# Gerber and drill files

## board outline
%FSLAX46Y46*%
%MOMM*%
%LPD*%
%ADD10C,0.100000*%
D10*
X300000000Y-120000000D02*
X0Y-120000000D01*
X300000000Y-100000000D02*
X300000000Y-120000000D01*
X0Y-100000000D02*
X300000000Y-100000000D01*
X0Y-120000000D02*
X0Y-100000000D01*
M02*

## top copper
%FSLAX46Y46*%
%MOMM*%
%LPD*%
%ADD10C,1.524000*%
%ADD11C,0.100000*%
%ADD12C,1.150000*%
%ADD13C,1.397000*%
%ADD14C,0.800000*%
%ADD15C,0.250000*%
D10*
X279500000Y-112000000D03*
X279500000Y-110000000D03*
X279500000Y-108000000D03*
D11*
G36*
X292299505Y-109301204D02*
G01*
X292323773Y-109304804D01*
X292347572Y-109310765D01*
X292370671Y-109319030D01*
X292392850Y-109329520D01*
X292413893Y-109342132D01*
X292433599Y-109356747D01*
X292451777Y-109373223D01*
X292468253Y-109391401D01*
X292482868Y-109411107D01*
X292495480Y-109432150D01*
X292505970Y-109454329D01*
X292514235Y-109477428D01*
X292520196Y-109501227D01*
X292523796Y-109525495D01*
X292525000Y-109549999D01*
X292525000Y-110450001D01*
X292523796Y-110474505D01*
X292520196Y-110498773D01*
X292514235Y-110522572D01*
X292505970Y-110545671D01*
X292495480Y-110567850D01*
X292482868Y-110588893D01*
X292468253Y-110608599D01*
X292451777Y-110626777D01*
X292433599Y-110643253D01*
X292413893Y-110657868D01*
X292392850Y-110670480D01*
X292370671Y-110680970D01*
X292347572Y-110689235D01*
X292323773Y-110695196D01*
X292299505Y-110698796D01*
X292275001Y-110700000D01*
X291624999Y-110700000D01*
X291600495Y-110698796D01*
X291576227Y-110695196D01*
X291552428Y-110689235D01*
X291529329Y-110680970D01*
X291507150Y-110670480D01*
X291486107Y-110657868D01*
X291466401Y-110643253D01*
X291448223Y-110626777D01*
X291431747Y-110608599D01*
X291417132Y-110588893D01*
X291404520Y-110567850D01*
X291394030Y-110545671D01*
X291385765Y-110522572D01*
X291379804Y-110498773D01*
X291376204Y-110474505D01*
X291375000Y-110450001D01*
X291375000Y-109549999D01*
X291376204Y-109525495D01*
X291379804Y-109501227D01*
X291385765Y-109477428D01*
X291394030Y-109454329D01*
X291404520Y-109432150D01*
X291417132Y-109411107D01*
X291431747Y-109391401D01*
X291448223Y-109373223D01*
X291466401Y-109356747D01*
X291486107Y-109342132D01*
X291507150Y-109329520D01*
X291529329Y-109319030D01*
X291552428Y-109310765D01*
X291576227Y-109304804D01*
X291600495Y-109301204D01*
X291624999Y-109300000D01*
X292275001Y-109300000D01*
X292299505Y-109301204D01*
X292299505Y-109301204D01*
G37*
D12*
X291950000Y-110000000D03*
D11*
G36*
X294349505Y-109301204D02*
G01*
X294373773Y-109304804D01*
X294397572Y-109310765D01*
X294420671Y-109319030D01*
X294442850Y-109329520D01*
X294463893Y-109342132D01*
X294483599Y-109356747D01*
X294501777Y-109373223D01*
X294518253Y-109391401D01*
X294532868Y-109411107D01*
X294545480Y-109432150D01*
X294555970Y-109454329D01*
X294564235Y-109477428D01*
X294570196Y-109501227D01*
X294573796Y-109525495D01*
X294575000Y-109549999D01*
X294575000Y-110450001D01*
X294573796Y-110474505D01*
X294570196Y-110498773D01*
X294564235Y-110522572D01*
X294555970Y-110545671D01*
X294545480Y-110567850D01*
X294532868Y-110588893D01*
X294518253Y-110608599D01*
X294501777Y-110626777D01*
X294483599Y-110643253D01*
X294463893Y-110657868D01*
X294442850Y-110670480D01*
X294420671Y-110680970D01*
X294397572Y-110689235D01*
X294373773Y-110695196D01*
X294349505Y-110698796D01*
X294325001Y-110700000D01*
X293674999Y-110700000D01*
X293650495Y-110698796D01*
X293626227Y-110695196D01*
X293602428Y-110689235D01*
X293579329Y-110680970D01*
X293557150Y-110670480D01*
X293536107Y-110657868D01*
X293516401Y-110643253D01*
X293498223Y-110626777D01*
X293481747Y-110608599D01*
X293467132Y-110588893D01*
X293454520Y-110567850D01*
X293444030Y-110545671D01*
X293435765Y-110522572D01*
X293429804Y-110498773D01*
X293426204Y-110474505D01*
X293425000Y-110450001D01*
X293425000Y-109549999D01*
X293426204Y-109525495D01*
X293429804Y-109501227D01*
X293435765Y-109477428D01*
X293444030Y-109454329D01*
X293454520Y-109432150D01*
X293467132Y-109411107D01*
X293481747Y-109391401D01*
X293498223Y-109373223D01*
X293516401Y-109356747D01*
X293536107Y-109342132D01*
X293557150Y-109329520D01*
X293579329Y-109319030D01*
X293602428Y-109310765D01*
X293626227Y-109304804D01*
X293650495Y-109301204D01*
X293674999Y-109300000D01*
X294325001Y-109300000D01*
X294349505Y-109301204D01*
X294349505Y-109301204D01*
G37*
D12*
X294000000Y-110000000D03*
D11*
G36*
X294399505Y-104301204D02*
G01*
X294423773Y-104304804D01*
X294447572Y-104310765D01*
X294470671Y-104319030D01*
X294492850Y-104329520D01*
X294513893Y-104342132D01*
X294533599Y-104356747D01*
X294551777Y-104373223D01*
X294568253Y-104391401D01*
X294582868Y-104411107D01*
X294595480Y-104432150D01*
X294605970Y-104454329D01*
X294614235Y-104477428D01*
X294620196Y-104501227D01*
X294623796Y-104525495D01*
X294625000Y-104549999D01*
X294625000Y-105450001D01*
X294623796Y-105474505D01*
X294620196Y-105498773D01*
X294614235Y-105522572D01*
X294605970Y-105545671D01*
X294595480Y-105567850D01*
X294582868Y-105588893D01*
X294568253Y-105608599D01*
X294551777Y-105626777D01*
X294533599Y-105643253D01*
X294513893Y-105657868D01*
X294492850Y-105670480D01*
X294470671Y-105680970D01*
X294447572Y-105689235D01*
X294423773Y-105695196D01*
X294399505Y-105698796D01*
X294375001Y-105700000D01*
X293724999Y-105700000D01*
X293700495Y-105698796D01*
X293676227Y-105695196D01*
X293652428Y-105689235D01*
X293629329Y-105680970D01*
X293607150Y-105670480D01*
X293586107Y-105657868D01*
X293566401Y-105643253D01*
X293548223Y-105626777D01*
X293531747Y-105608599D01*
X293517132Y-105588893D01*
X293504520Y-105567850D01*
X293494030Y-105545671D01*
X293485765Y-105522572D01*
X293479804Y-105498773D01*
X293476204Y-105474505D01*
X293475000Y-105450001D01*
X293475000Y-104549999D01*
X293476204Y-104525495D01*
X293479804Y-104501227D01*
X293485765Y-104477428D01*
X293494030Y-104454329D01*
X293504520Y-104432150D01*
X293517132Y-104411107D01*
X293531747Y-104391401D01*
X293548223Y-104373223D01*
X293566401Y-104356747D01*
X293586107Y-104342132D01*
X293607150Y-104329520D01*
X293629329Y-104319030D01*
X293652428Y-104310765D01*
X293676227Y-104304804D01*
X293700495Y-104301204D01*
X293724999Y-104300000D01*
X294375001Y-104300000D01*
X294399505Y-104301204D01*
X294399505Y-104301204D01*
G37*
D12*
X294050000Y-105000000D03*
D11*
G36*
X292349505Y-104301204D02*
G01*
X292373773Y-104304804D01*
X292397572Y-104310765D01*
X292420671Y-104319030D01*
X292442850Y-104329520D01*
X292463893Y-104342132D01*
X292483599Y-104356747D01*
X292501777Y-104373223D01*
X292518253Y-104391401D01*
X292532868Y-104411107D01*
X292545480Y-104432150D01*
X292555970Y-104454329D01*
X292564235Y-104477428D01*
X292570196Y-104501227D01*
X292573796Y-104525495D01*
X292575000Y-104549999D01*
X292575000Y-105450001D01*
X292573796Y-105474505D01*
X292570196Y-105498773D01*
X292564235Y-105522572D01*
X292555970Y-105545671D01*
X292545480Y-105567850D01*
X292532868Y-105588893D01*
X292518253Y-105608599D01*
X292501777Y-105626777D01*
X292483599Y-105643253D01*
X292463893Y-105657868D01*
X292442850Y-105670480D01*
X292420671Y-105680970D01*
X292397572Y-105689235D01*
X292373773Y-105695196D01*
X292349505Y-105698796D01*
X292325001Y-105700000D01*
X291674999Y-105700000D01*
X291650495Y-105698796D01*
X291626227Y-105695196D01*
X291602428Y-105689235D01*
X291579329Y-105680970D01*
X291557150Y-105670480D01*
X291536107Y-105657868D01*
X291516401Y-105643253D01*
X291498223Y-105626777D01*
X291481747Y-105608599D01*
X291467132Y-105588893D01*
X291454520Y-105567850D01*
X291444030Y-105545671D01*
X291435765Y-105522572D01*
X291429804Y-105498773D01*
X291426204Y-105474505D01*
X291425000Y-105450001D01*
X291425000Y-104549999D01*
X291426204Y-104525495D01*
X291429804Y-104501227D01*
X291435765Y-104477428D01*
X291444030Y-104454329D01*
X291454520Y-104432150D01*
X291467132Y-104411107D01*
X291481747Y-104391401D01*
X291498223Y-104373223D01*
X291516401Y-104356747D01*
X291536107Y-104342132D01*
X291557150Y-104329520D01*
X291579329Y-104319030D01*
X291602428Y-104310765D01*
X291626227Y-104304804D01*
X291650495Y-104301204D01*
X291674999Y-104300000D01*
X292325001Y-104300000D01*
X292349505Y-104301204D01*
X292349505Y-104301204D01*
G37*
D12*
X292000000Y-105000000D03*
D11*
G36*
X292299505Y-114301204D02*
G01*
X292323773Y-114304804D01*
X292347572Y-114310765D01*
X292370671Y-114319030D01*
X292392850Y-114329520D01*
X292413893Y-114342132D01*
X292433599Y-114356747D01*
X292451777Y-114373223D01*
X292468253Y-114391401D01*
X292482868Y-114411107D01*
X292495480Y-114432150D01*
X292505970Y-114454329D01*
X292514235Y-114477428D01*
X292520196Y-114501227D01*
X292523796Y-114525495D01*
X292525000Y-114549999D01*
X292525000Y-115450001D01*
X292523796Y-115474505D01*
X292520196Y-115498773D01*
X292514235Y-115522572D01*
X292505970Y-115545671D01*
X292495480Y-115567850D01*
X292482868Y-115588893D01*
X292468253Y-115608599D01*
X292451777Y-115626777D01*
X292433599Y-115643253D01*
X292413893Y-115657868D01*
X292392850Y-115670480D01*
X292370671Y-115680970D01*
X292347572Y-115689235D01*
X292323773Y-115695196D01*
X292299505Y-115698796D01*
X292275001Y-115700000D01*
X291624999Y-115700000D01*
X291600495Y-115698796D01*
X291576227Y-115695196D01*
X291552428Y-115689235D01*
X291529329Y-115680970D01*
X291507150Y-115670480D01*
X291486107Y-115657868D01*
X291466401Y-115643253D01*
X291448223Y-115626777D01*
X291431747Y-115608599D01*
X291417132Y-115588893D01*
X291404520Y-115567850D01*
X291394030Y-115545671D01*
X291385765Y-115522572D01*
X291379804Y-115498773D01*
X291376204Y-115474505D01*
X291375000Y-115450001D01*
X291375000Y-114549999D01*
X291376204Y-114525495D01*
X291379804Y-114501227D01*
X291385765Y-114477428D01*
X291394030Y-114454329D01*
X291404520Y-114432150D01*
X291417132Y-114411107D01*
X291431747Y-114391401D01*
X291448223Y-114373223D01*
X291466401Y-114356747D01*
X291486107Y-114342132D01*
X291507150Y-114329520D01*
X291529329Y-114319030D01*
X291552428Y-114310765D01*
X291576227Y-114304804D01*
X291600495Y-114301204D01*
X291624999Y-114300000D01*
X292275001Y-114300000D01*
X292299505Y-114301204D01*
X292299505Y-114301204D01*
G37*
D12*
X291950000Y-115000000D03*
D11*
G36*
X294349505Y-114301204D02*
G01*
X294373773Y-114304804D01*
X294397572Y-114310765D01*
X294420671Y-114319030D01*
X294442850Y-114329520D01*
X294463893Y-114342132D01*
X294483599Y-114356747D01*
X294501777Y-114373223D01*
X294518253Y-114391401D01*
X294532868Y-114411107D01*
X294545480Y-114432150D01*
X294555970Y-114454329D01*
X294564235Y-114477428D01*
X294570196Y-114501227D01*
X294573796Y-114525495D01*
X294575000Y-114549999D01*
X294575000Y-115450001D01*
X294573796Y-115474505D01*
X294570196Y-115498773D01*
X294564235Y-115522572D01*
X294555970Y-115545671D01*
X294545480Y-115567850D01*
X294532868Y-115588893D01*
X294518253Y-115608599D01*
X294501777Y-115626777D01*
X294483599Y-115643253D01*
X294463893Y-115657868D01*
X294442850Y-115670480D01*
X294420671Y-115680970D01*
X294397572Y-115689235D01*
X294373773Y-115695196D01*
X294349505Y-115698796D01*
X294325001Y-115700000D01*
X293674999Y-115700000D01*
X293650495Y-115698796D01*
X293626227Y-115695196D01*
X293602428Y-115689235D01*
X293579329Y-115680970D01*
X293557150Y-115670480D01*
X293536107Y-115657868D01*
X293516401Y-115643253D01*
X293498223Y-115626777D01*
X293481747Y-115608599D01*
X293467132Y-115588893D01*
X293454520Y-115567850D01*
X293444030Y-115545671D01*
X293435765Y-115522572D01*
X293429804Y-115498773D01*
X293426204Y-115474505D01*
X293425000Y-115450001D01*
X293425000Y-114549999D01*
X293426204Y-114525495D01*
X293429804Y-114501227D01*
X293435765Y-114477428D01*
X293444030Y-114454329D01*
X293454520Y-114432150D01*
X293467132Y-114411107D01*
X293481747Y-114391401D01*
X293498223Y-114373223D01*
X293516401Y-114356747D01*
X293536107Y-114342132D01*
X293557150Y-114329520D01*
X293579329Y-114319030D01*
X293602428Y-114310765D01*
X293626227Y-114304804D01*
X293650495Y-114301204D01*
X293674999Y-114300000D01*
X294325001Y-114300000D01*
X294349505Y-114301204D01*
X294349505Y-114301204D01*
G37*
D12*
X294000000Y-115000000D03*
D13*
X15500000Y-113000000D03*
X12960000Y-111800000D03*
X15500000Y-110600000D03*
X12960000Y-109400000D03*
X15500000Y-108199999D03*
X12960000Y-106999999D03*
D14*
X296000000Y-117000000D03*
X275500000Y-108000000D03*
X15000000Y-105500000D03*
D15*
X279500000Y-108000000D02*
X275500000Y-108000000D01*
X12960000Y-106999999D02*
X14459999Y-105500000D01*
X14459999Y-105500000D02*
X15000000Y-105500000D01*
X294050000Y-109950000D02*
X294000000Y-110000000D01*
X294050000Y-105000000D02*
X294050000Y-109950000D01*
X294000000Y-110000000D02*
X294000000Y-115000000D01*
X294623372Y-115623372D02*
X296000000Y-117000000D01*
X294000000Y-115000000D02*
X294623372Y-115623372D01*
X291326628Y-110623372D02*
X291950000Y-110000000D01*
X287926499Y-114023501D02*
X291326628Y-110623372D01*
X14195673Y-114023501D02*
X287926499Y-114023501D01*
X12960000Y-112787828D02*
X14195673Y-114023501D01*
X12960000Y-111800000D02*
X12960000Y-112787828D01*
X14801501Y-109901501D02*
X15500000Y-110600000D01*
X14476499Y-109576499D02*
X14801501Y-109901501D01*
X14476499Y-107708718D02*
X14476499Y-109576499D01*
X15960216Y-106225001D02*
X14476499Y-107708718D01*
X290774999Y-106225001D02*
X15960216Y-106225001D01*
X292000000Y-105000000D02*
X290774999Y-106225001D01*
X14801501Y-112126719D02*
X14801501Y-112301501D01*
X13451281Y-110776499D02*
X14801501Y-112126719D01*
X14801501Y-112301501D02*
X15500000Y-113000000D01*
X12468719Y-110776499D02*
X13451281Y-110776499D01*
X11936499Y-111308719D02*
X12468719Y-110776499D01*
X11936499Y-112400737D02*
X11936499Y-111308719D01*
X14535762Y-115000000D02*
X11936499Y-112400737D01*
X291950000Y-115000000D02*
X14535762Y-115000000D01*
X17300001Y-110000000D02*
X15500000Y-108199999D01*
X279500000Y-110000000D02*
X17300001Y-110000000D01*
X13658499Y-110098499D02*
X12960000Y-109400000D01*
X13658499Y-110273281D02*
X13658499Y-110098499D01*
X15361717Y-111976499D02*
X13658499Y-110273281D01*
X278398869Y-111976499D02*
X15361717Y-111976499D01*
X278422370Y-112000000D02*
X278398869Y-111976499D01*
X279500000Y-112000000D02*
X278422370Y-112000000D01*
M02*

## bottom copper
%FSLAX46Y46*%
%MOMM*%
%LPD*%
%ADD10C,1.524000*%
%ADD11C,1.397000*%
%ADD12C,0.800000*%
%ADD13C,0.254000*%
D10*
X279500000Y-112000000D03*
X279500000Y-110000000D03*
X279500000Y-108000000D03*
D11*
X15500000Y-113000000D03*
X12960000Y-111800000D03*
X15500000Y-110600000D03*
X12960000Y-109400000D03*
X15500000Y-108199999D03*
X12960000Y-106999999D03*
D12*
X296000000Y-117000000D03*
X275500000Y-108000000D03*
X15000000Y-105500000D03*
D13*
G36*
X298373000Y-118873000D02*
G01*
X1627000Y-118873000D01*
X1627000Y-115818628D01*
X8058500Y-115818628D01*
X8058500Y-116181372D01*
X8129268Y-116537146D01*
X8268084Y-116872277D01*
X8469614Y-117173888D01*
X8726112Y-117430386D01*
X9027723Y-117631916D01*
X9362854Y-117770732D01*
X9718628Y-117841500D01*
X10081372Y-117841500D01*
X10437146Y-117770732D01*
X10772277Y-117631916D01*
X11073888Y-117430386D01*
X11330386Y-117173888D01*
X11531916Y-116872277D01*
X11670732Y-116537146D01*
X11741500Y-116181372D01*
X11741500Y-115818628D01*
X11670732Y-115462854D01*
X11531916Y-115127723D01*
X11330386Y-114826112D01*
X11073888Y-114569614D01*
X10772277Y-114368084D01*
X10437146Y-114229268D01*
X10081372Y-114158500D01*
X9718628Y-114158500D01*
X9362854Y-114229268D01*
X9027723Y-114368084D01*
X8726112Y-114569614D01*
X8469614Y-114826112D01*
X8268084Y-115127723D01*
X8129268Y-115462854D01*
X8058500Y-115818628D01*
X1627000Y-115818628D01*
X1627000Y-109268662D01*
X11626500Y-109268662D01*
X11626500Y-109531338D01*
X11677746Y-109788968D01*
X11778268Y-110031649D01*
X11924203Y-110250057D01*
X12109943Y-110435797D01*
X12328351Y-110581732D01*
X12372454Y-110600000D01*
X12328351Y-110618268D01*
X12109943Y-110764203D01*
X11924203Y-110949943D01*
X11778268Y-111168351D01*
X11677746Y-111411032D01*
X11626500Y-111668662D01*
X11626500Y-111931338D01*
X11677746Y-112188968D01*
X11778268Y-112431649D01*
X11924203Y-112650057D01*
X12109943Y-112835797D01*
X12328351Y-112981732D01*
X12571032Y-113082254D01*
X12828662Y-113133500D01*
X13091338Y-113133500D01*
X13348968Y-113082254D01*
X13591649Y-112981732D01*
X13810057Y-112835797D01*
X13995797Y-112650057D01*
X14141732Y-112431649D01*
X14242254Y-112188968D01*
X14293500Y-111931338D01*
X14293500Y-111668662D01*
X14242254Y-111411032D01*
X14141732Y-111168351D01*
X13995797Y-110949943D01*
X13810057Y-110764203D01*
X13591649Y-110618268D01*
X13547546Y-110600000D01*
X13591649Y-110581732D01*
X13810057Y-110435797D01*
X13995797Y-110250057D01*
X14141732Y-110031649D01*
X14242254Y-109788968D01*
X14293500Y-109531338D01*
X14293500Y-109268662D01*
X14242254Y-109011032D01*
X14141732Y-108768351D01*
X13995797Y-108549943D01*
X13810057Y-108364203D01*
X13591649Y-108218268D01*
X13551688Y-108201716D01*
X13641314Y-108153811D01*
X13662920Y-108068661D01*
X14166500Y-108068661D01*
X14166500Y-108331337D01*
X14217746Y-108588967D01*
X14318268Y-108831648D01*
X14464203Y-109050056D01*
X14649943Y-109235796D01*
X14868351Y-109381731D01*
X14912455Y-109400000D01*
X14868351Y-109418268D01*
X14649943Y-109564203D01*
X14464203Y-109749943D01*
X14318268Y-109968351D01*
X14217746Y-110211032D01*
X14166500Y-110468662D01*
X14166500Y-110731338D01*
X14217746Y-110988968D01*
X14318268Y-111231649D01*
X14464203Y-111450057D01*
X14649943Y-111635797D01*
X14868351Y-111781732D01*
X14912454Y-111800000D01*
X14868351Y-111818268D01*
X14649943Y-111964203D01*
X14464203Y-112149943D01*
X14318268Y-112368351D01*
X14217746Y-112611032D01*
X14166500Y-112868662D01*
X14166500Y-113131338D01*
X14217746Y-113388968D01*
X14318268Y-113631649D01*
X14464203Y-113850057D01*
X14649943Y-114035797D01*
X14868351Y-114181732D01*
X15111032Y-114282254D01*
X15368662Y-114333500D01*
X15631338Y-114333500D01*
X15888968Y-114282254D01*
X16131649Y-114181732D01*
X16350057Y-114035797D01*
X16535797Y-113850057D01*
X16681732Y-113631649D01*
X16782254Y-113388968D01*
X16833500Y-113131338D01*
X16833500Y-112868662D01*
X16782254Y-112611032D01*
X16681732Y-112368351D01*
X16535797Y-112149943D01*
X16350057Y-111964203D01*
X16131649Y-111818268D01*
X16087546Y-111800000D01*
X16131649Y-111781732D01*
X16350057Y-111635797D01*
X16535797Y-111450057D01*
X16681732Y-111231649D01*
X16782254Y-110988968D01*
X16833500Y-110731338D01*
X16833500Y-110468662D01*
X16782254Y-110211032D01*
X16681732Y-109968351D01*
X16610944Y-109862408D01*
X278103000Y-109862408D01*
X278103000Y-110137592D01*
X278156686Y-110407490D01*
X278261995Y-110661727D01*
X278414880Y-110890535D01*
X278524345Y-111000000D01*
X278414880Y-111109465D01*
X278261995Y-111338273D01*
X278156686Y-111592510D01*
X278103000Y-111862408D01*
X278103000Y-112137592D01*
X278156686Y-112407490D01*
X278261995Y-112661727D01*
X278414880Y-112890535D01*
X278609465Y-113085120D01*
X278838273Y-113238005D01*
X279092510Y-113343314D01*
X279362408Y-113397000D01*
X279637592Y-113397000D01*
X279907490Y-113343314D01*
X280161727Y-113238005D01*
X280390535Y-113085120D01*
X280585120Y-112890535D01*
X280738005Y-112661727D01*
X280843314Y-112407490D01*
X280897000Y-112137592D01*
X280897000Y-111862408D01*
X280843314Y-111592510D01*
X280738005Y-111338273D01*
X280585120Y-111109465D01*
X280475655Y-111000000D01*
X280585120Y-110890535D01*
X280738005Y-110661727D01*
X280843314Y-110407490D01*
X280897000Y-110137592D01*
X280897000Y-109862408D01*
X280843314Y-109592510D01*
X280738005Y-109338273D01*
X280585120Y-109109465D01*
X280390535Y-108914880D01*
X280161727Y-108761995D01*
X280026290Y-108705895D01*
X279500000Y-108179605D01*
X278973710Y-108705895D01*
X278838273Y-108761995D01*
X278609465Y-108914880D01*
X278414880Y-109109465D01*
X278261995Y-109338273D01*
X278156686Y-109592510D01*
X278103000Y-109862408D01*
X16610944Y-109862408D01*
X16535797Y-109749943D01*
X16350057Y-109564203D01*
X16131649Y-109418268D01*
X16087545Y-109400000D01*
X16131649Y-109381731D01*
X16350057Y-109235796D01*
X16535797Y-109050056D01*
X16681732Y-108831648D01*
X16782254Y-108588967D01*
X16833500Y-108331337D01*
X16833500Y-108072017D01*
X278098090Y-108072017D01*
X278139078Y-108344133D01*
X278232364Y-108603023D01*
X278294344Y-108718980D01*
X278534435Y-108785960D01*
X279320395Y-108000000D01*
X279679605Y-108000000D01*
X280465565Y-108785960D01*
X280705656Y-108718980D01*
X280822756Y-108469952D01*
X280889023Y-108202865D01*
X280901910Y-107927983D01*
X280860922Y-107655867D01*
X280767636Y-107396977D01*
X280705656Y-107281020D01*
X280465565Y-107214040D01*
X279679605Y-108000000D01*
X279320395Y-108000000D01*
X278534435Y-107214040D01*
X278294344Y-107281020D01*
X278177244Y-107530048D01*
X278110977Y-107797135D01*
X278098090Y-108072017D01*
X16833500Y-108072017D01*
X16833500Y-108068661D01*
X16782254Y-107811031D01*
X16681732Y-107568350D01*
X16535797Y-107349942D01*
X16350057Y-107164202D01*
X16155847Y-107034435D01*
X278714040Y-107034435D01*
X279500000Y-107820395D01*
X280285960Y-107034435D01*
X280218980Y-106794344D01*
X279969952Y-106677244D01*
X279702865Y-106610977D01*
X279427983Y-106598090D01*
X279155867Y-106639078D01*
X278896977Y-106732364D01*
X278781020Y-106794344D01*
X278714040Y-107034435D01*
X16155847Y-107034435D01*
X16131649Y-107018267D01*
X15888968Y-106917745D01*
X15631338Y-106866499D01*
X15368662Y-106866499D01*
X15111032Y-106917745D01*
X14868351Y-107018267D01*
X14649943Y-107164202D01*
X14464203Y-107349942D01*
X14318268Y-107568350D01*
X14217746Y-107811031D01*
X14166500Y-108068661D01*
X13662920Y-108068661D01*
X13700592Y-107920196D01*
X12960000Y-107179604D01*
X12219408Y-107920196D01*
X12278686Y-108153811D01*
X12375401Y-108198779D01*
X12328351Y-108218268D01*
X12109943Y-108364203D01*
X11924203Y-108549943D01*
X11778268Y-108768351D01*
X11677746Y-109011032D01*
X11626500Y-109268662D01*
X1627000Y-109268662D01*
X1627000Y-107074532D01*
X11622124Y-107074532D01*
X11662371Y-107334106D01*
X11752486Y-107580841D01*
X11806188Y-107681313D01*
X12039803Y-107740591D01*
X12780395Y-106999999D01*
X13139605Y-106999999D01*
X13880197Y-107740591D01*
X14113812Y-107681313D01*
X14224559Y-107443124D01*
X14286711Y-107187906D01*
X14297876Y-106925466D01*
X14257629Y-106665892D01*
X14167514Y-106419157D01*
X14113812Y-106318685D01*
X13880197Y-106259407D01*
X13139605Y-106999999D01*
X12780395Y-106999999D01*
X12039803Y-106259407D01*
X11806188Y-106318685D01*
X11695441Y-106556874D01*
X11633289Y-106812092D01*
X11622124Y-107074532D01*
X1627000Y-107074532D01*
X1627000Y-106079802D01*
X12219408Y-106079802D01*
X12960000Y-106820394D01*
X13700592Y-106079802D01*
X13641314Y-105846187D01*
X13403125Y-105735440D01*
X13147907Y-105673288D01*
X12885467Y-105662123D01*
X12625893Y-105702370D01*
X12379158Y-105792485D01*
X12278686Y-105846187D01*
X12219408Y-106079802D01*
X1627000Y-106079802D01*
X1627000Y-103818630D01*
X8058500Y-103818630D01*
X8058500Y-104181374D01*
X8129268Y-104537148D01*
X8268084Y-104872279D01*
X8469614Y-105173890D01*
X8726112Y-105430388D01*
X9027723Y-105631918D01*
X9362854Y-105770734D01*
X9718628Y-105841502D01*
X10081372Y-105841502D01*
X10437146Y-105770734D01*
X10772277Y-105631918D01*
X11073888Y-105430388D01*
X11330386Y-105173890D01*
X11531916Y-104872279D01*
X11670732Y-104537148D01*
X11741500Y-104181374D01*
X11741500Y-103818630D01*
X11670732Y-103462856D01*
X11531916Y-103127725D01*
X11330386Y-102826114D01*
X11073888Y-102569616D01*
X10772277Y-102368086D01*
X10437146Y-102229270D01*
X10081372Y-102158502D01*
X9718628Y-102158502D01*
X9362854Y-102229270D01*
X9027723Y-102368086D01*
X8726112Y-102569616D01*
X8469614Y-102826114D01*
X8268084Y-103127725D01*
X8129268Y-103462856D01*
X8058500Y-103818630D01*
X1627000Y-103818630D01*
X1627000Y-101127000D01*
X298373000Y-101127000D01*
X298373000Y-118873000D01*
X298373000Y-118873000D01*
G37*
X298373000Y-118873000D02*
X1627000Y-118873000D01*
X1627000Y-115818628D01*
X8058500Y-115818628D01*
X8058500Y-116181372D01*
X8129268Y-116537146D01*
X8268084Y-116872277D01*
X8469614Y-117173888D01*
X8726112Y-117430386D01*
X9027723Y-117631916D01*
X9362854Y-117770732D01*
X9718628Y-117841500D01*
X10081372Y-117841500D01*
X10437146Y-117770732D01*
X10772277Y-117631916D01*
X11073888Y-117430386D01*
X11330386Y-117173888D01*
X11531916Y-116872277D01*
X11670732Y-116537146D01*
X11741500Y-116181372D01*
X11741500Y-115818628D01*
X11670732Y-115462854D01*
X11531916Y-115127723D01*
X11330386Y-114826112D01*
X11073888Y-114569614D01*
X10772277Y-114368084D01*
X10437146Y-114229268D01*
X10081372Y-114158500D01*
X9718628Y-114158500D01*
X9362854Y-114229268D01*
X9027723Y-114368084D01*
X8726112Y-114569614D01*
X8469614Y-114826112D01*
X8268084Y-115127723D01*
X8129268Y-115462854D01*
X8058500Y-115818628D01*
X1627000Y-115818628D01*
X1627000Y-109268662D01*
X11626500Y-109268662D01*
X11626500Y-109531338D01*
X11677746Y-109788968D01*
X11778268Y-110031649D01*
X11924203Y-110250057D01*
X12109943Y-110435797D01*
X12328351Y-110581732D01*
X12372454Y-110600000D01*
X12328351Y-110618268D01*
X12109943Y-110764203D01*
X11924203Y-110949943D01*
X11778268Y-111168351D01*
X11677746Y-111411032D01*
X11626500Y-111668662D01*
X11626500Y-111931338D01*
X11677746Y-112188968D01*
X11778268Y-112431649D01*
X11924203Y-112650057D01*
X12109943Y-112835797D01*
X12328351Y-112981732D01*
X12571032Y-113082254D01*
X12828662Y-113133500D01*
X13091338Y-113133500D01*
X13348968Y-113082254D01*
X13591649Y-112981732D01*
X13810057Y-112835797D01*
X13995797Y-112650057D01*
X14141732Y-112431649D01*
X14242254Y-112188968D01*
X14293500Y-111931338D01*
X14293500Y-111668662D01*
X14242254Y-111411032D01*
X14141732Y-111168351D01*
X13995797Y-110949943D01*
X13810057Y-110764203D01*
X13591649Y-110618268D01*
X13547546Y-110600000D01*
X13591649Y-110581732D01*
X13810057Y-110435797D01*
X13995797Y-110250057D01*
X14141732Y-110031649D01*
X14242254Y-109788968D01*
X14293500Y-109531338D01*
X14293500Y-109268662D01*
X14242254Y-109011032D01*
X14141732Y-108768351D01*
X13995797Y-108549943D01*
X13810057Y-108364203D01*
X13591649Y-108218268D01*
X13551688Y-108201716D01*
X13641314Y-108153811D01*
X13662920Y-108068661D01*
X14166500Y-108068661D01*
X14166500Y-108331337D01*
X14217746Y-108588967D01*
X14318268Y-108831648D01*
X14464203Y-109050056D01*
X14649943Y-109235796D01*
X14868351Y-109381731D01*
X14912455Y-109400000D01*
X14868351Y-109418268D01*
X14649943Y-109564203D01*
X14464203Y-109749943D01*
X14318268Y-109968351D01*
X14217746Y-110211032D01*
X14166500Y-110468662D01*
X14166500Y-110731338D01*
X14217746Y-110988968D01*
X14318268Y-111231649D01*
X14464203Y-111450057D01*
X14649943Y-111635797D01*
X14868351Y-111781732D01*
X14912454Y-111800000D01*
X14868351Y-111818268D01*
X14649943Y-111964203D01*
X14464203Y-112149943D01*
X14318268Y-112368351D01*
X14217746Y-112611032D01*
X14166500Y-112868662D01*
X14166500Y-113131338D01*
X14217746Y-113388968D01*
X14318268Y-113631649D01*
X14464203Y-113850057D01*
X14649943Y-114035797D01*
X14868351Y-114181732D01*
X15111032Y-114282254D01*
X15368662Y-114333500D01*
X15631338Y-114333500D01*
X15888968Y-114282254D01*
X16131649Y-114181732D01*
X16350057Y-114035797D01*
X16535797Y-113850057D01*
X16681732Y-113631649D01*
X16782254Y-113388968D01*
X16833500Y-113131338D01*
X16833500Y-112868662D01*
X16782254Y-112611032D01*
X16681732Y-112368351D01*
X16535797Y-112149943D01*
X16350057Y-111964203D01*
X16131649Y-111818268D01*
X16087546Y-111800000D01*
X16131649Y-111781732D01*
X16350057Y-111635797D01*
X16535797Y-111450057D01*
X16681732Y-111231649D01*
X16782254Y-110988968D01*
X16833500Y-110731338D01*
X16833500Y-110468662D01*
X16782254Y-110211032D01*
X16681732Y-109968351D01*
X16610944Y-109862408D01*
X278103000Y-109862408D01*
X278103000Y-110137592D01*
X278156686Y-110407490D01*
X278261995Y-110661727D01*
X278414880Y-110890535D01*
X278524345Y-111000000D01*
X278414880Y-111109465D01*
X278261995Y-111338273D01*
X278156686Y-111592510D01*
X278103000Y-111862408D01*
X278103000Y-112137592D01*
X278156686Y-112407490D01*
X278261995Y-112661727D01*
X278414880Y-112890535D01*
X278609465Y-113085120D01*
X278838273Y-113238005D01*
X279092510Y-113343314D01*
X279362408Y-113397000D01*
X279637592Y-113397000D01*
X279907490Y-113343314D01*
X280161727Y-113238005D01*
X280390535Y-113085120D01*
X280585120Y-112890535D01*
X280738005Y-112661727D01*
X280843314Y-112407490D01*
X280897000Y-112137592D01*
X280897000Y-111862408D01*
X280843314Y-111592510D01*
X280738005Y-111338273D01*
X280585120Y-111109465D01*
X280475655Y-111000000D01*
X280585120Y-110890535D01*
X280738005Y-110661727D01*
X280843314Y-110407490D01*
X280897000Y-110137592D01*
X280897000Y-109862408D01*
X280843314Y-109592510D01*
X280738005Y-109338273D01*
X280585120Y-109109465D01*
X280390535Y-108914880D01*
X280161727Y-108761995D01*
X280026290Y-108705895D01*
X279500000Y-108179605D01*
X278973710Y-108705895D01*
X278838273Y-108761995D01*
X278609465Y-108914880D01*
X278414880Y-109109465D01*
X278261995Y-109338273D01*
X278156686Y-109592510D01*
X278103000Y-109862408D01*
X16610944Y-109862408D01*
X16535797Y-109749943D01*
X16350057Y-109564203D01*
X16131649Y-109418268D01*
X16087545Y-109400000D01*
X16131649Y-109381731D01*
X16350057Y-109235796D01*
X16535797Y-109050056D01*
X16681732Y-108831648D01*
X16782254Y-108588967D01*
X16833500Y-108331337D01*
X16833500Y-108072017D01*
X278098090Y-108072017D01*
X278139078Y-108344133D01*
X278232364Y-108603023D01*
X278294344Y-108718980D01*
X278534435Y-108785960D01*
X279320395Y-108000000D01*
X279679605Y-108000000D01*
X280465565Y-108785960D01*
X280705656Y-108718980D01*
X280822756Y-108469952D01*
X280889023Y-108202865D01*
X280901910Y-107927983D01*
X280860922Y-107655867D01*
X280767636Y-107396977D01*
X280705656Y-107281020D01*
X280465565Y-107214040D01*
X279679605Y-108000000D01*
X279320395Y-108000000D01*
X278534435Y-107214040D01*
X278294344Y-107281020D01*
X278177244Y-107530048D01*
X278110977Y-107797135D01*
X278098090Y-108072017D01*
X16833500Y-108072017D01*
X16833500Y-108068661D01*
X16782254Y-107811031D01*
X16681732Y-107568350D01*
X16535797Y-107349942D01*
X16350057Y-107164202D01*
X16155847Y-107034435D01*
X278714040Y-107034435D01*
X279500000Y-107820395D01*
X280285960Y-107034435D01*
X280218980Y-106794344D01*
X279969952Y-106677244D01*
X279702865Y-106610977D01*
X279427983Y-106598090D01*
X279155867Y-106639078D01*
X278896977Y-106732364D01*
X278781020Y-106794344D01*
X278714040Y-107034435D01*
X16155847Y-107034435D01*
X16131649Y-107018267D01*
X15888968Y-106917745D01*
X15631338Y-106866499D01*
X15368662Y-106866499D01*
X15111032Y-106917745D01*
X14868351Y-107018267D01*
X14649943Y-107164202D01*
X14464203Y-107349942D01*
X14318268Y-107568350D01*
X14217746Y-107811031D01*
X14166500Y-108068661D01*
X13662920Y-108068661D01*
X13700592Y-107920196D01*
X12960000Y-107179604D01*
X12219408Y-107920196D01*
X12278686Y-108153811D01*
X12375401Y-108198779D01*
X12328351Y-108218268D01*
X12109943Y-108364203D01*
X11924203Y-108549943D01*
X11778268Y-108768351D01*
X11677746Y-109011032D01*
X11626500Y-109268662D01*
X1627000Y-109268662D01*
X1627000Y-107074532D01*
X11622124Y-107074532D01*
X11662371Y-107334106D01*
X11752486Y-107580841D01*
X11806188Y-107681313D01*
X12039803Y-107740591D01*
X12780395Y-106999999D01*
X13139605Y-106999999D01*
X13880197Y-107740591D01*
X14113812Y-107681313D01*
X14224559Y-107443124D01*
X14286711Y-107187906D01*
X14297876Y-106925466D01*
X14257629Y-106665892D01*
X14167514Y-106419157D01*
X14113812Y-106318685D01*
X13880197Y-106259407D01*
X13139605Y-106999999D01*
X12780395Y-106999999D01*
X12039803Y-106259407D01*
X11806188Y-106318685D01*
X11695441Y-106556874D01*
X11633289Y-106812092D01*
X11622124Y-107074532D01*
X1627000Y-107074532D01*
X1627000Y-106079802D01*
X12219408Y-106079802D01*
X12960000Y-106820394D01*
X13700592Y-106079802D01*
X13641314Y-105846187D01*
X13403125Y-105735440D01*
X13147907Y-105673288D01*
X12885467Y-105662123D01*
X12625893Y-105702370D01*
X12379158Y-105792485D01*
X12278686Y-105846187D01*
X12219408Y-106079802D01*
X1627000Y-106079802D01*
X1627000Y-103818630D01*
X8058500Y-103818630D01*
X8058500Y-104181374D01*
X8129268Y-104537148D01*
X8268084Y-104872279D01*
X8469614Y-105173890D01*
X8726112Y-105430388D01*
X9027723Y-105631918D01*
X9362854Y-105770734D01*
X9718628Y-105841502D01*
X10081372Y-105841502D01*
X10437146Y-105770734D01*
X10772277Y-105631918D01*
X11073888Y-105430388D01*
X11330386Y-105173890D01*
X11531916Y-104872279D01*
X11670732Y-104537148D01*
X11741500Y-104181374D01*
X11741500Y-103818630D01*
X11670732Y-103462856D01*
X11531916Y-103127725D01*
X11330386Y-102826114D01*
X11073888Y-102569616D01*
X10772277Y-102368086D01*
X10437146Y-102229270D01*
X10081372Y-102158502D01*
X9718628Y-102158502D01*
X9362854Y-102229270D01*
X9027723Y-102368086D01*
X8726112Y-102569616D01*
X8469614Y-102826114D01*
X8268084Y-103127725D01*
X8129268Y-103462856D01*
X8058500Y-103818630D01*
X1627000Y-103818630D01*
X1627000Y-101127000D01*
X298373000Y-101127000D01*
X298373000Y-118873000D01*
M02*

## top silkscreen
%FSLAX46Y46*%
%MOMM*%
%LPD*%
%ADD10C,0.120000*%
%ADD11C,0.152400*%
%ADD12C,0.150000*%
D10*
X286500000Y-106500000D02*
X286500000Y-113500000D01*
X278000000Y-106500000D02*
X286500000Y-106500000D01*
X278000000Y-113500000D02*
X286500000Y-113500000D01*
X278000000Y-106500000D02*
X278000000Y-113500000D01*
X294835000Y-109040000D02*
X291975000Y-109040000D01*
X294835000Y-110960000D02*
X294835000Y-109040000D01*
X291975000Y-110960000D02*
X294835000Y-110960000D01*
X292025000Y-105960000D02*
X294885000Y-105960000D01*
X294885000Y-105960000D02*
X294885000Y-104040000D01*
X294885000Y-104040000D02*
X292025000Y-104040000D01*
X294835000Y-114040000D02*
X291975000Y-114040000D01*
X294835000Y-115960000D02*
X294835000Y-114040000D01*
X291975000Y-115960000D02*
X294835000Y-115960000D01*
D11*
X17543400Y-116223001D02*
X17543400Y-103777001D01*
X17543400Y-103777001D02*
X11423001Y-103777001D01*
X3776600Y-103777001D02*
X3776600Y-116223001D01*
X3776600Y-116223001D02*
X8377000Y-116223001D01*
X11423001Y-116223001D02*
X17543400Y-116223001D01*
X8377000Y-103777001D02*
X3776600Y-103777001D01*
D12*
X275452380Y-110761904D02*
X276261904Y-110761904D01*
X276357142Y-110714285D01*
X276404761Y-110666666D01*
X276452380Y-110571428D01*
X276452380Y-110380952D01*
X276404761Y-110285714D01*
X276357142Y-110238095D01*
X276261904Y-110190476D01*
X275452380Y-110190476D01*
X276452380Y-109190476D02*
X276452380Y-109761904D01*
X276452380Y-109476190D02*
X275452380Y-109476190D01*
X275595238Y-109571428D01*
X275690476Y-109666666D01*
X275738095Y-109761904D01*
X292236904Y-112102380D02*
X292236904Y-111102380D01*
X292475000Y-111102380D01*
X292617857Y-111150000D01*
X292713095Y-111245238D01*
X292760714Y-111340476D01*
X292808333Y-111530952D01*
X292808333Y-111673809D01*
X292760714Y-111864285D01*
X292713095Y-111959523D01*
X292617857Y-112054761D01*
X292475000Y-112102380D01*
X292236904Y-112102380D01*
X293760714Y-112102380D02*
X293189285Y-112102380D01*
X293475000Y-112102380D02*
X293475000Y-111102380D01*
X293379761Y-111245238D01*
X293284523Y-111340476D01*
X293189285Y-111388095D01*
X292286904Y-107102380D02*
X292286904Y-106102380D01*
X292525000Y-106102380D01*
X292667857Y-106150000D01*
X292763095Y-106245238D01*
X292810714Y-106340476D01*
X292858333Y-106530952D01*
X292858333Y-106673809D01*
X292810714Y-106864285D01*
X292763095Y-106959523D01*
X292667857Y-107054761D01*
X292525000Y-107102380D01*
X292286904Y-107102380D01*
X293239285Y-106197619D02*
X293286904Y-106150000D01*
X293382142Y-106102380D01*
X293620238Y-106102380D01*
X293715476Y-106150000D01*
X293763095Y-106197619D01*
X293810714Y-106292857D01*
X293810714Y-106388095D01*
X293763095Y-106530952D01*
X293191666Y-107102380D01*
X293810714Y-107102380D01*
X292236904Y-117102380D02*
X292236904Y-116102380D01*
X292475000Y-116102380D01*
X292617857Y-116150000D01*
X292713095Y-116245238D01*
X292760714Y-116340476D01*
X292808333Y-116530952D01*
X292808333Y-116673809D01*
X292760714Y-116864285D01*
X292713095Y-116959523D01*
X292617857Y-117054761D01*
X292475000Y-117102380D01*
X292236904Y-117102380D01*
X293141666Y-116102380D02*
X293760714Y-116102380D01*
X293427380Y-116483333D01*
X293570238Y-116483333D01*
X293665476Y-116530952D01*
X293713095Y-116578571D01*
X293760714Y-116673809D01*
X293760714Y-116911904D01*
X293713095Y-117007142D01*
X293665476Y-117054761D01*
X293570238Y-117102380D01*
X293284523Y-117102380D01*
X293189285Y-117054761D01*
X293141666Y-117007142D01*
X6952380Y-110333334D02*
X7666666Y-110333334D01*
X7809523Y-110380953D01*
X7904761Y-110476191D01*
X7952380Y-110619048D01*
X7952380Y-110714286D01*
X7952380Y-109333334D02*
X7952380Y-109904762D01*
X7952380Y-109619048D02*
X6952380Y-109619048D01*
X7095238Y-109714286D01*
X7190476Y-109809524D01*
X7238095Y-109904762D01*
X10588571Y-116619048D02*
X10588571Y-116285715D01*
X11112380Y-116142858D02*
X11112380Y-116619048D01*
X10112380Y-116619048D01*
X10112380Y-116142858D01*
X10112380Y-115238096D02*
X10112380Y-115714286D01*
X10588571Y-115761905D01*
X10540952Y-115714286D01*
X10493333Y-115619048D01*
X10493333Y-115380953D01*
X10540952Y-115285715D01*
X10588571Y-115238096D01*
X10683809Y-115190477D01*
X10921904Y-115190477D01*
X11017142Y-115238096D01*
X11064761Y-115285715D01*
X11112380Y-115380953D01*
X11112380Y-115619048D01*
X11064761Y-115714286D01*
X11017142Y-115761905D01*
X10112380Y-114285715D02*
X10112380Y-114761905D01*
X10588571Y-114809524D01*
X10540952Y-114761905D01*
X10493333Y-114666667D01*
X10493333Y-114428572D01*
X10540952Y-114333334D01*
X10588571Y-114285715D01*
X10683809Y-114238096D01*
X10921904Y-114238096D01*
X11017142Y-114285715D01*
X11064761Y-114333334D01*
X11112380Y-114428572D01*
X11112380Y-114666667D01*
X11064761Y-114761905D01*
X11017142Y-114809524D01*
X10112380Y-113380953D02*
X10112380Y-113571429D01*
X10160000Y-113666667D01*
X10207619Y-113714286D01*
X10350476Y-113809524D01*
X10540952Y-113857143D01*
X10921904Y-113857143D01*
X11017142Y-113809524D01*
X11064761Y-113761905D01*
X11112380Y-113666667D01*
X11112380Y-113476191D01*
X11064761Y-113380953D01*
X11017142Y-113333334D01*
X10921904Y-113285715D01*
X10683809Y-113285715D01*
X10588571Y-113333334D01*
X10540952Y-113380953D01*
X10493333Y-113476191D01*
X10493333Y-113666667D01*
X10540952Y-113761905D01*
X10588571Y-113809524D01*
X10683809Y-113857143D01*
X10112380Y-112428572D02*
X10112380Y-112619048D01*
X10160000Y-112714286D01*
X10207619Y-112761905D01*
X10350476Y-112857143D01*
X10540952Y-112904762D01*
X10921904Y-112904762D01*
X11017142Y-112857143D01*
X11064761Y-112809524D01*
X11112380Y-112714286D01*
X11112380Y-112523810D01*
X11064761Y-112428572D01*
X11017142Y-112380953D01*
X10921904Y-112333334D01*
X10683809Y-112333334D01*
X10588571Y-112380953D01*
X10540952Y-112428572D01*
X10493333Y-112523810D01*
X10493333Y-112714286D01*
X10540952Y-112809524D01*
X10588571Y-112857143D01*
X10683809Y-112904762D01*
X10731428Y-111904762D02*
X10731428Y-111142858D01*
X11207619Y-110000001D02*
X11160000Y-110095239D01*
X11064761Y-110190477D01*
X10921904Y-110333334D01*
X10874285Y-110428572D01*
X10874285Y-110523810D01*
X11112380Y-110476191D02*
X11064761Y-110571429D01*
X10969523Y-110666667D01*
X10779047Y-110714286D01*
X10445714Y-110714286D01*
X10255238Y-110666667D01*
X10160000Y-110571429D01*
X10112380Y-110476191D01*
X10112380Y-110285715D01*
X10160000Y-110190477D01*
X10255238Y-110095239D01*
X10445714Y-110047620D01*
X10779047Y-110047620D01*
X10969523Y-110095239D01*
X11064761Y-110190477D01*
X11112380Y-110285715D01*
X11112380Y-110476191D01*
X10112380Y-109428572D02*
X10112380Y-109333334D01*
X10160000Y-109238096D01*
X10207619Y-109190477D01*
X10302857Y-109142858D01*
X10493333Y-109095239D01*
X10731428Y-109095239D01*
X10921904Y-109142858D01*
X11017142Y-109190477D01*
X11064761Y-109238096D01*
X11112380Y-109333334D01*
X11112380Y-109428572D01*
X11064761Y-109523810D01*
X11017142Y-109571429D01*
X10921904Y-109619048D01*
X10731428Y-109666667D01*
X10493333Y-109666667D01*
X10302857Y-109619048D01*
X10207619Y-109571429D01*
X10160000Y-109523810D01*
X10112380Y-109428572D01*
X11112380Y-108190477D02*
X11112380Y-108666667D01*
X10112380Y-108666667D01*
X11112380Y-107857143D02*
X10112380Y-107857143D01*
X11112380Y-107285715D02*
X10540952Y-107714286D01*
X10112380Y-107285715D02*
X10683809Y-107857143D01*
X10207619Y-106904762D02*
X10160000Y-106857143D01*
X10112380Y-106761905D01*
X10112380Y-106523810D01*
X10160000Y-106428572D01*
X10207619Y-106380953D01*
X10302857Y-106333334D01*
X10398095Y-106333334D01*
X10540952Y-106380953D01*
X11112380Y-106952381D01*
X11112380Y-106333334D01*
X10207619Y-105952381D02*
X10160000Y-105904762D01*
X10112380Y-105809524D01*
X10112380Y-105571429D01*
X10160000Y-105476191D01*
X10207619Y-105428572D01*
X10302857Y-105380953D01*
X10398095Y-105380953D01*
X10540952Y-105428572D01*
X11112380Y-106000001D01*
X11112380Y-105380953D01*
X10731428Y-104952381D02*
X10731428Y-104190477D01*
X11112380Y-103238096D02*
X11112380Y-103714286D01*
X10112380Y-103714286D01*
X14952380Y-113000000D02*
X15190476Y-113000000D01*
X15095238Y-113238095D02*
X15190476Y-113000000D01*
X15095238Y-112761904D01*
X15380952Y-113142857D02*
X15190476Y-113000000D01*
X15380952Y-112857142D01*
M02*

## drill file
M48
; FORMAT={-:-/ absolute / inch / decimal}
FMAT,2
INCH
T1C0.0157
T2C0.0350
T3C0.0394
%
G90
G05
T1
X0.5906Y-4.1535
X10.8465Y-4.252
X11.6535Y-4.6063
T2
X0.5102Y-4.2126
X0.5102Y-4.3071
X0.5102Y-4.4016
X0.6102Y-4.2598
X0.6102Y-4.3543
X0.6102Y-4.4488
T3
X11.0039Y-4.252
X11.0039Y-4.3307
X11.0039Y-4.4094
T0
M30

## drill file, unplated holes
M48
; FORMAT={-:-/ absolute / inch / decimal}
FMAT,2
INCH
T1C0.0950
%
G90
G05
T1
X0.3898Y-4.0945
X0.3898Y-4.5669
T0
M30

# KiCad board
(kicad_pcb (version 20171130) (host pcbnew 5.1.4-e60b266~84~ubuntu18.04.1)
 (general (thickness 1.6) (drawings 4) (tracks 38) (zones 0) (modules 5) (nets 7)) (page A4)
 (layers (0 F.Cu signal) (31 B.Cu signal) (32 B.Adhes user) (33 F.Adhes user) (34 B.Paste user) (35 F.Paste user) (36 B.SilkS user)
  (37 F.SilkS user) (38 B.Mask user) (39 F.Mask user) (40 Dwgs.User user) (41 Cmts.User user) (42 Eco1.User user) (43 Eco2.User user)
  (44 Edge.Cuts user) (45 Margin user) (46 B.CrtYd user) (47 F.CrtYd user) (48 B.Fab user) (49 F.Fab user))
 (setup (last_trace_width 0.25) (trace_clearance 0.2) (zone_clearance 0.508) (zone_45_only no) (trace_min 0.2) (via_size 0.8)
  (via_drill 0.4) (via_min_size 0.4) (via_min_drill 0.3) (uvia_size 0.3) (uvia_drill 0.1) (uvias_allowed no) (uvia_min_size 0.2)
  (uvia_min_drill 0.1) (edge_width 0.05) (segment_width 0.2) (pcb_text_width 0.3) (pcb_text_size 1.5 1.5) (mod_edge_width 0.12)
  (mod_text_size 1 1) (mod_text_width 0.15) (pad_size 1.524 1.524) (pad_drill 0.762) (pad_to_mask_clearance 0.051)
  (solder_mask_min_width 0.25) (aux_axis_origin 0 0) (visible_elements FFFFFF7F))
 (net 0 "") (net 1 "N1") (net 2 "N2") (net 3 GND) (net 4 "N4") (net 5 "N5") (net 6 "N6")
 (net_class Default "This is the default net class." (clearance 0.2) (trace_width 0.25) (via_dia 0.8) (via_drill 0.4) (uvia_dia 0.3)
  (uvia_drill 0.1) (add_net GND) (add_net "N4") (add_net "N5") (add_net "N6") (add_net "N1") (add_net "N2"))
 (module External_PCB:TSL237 (layer F.Cu) (at 276.5 110 270)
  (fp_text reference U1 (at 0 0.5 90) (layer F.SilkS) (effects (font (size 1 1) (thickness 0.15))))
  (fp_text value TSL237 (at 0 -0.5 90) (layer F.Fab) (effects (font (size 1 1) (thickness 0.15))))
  (fp_line (start -3.5 -10) (end 3.5 -10) (layer F.SilkS) (width 0.12))
  (fp_line (start -3.5 -1.5) (end -3.5 -10) (layer F.SilkS) (width 0.12))
  (fp_line (start 3.5 -1.5) (end 3.5 -10) (layer F.SilkS) (width 0.12))
  (fp_line (start -3.5 -1.5) (end 3.5 -1.5) (layer F.SilkS) (width 0.12))
  (pad 3 thru_hole circle (at 2 -3 270) (size 1.524 1.524) (drill 1) (layers *.Cu *.Mask) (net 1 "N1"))
  (pad 2 thru_hole circle (at 0 -3 270) (size 1.524 1.524) (drill 1) (layers *.Cu *.Mask) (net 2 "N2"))
  (pad 1 thru_hole circle (at -2 -3 270) (size 1.524 1.524) (drill 1) (layers *.Cu *.Mask) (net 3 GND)))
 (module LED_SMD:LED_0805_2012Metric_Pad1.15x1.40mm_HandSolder (layer F.Cu) (at 292.975 110 180)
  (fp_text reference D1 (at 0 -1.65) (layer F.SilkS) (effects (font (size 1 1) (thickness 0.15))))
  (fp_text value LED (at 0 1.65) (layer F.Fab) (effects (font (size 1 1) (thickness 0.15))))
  (fp_line (start -1.86 0.96) (end 1 0.96) (layer F.SilkS) (width 0.12))
  (fp_line (start -1.86 -0.96) (end -1.86 0.96) (layer F.SilkS) (width 0.12))
  (fp_line (start 1 -0.96) (end -1.86 -0.96) (layer F.SilkS) (width 0.12))
  (pad 2 smd roundrect (at 1.025 0 180) (size 1.15 1.4) (layers F.Cu F.Paste F.Mask) (roundrect_rratio 0.217391) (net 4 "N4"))
  (pad 1 smd roundrect (at -1.025 0 180) (size 1.15 1.4) (layers F.Cu F.Paste F.Mask) (roundrect_rratio 0.217391) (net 3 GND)))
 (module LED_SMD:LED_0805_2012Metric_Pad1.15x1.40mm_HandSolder (layer F.Cu) (at 293.025 105 180)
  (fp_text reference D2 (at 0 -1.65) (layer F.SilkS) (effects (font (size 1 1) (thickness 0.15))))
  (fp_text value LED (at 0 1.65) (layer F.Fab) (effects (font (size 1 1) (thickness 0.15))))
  (fp_line (start 1 -0.96) (end -1.86 -0.96) (layer F.SilkS) (width 0.12))
  (fp_line (start -1.86 -0.96) (end -1.86 0.96) (layer F.SilkS) (width 0.12))
  (fp_line (start -1.86 0.96) (end 1 0.96) (layer F.SilkS) (width 0.12))
  (pad 1 smd roundrect (at -1.025 0 180) (size 1.15 1.4) (layers F.Cu F.Paste F.Mask) (roundrect_rratio 0.217391) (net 3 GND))
  (pad 2 smd roundrect (at 1.025 0 180) (size 1.15 1.4) (layers F.Cu F.Paste F.Mask) (roundrect_rratio 0.217391) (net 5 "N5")))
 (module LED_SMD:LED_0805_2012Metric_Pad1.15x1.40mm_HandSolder (layer F.Cu) (at 292.975 115 180)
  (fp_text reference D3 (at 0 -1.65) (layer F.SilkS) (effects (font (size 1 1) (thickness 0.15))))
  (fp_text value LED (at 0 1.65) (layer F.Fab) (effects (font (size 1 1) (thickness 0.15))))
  (fp_line (start -1.86 0.96) (end 1 0.96) (layer F.SilkS) (width 0.12))
  (fp_line (start -1.86 -0.96) (end -1.86 0.96) (layer F.SilkS) (width 0.12))
  (fp_line (start 1 -0.96) (end -1.86 -0.96) (layer F.SilkS) (width 0.12))
  (pad 2 smd roundrect (at 1.025 0 180) (size 1.15 1.4) (layers F.Cu F.Paste F.Mask) (roundrect_rratio 0.217391) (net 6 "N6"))
  (pad 1 smd roundrect (at -1.025 0 180) (size 1.15 1.4) (layers F.Cu F.Paste F.Mask) (roundrect_rratio 0.217391) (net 3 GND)))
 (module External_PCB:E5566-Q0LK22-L (layer F.Cu) (at 15.5 113 90)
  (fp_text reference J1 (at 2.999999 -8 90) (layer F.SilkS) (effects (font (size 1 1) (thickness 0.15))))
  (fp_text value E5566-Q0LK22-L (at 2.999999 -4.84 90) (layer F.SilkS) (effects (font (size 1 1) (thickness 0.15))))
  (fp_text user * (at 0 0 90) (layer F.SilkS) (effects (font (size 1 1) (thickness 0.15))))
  (fp_line (start -3.223001 2.0434) (end 9.222999 2.0434) (layer F.SilkS) (width 0.1524))
  (fp_line (start 9.222999 2.0434) (end 9.222999 -4.076999) (layer F.SilkS) (width 0.1524))
  (fp_line (start 9.222999 -11.7234) (end -3.223001 -11.7234) (layer F.SilkS) (width 0.1524))
  (fp_line (start -3.223001 -11.7234) (end -3.223001 -7.123) (layer F.SilkS) (width 0.1524))
  (fp_line (start -3.223001 -4.076999) (end -3.223001 2.0434) (layer F.SilkS) (width 0.1524))
  (fp_line (start 9.222999 -7.123) (end 9.222999 -11.7234) (layer F.SilkS) (width 0.1524))
  (pad 1 thru_hole circle (at 0 0 90) (size 1.397 1.397) (drill 0.889) (layers *.Cu *.Mask) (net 6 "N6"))
  (pad 2 thru_hole circle (at 1.2 -2.54 90) (size 1.397 1.397) (drill 0.889) (layers *.Cu *.Mask) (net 4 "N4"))
  (pad 3 thru_hole circle (at 2.4 0 90) (size 1.397 1.397) (drill 0.889) (layers *.Cu *.Mask) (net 5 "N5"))
  (pad 4 thru_hole circle (at 3.6 -2.54 90) (size 1.397 1.397) (drill 0.889) (layers *.Cu *.Mask) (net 1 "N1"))
  (pad 5 thru_hole circle (at 4.800001 0 90) (size 1.397 1.397) (drill 0.889) (layers *.Cu *.Mask) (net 2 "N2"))
  (pad 6 thru_hole circle (at 6.000001 -2.54 90) (size 1.397 1.397) (drill 0.889) (layers *.Cu *.Mask) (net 3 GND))
  (pad 7 np_thru_hole circle (at -3 -5.6 90) (size 2.413 2.413) (drill 2.413) (layers *.Cu *.Mask))
  (pad 8 np_thru_hole circle (at 8.999998 -5.6 90) (size 2.413 2.413) (drill 2.413) (layers *.Cu *.Mask)))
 (gr_line (start 300 120) (end 0 120) (layer Edge.Cuts) (width 0.1))
 (gr_line (start 300 100) (end 300 120) (layer Edge.Cuts) (width 0.1))
 (gr_line (start 0 100) (end 300 100) (layer Edge.Cuts) (width 0.1))
 (gr_line (start 0 120) (end 0 100) (layer Edge.Cuts) (width 0.1))
 (via (at 296 117) (size 0.8) (drill 0.4) (layers F.Cu B.Cu) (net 3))
 (via (at 275.5 108) (size 0.8) (drill 0.4) (layers F.Cu B.Cu) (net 3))
 (segment (start 279.5 108) (end 275.5 108) (width 0.25) (layer F.Cu) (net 3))
 (via (at 15 105.5) (size 0.8) (drill 0.4) (layers F.Cu B.Cu) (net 3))
 (segment (start 12.96 106.999999) (end 14.459999 105.5) (width 0.25) (layer F.Cu) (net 3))
 (segment (start 14.459999 105.5) (end 15 105.5) (width 0.25) (layer F.Cu) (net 3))
 (segment (start 294.05 109.95) (end 294 110) (width 0.25) (layer F.Cu) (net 3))
 (segment (start 294.05 105) (end 294.05 109.95) (width 0.25) (layer F.Cu) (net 3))
 (segment (start 294 110) (end 294 115) (width 0.25) (layer F.Cu) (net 3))
 (segment (start 294.623372 115.623372) (end 296 117) (width 0.25) (layer F.Cu) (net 3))
 (segment (start 294 115) (end 294.623372 115.623372) (width 0.25) (layer F.Cu) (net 3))
 (segment (start 291.326628 110.623372) (end 291.95 110) (width 0.25) (layer F.Cu) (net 4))
 (segment (start 287.926499 114.023501) (end 291.326628 110.623372) (width 0.25) (layer F.Cu) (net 4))
 (segment (start 14.195673 114.023501) (end 287.926499 114.023501) (width 0.25) (layer F.Cu) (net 4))
 (segment (start 12.96 112.787828) (end 14.195673 114.023501) (width 0.25) (layer F.Cu) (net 4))
 (segment (start 12.96 111.8) (end 12.96 112.787828) (width 0.25) (layer F.Cu) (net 4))
 (segment (start 14.801501 109.901501) (end 15.5 110.6) (width 0.25) (layer F.Cu) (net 5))
 (segment (start 14.476499 109.576499) (end 14.801501 109.901501) (width 0.25) (layer F.Cu) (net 5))
 (segment (start 14.476499 107.708718) (end 14.476499 109.576499) (width 0.25) (layer F.Cu) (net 5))
 (segment (start 15.960216 106.225001) (end 14.476499 107.708718) (width 0.25) (layer F.Cu) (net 5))
 (segment (start 290.774999 106.225001) (end 15.960216 106.225001) (width 0.25) (layer F.Cu) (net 5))
 (segment (start 292 105) (end 290.774999 106.225001) (width 0.25) (layer F.Cu) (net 5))
 (segment (start 14.801501 112.126719) (end 14.801501 112.301501) (width 0.25) (layer F.Cu) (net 6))
 (segment (start 13.451281 110.776499) (end 14.801501 112.126719) (width 0.25) (layer F.Cu) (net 6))
 (segment (start 14.801501 112.301501) (end 15.5 113) (width 0.25) (layer F.Cu) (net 6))
 (segment (start 12.468719 110.776499) (end 13.451281 110.776499) (width 0.25) (layer F.Cu) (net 6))
 (segment (start 11.936499 111.308719) (end 12.468719 110.776499) (width 0.25) (layer F.Cu) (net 6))
 (segment (start 11.936499 112.400737) (end 11.936499 111.308719) (width 0.25) (layer F.Cu) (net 6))
 (segment (start 14.535762 115) (end 11.936499 112.400737) (width 0.25) (layer F.Cu) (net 6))
 (segment (start 291.95 115) (end 14.535762 115) (width 0.25) (layer F.Cu) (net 6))
 (segment (start 17.300001 110) (end 15.5 108.199999) (width 0.25) (layer F.Cu) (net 2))
 (segment (start 279.5 110) (end 17.300001 110) (width 0.25) (layer F.Cu) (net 2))
 (segment (start 13.658499 110.098499) (end 12.96 109.4) (width 0.25) (layer F.Cu) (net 1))
 (segment (start 13.658499 110.273281) (end 13.658499 110.098499) (width 0.25) (layer F.Cu) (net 1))
 (segment (start 15.361717 111.976499) (end 13.658499 110.273281) (width 0.25) (layer F.Cu) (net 1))
 (segment (start 278.398869 111.976499) (end 15.361717 111.976499) (width 0.25) (layer F.Cu) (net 1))
 (segment (start 278.42237 112) (end 278.398869 111.976499) (width 0.25) (layer F.Cu) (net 1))
 (segment (start 279.5 112) (end 278.42237 112) (width 0.25) (layer F.Cu) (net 1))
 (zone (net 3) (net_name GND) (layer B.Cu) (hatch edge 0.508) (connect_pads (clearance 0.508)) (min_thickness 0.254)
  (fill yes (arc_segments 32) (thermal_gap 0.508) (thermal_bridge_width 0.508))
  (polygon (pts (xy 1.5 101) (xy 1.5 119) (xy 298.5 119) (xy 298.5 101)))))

